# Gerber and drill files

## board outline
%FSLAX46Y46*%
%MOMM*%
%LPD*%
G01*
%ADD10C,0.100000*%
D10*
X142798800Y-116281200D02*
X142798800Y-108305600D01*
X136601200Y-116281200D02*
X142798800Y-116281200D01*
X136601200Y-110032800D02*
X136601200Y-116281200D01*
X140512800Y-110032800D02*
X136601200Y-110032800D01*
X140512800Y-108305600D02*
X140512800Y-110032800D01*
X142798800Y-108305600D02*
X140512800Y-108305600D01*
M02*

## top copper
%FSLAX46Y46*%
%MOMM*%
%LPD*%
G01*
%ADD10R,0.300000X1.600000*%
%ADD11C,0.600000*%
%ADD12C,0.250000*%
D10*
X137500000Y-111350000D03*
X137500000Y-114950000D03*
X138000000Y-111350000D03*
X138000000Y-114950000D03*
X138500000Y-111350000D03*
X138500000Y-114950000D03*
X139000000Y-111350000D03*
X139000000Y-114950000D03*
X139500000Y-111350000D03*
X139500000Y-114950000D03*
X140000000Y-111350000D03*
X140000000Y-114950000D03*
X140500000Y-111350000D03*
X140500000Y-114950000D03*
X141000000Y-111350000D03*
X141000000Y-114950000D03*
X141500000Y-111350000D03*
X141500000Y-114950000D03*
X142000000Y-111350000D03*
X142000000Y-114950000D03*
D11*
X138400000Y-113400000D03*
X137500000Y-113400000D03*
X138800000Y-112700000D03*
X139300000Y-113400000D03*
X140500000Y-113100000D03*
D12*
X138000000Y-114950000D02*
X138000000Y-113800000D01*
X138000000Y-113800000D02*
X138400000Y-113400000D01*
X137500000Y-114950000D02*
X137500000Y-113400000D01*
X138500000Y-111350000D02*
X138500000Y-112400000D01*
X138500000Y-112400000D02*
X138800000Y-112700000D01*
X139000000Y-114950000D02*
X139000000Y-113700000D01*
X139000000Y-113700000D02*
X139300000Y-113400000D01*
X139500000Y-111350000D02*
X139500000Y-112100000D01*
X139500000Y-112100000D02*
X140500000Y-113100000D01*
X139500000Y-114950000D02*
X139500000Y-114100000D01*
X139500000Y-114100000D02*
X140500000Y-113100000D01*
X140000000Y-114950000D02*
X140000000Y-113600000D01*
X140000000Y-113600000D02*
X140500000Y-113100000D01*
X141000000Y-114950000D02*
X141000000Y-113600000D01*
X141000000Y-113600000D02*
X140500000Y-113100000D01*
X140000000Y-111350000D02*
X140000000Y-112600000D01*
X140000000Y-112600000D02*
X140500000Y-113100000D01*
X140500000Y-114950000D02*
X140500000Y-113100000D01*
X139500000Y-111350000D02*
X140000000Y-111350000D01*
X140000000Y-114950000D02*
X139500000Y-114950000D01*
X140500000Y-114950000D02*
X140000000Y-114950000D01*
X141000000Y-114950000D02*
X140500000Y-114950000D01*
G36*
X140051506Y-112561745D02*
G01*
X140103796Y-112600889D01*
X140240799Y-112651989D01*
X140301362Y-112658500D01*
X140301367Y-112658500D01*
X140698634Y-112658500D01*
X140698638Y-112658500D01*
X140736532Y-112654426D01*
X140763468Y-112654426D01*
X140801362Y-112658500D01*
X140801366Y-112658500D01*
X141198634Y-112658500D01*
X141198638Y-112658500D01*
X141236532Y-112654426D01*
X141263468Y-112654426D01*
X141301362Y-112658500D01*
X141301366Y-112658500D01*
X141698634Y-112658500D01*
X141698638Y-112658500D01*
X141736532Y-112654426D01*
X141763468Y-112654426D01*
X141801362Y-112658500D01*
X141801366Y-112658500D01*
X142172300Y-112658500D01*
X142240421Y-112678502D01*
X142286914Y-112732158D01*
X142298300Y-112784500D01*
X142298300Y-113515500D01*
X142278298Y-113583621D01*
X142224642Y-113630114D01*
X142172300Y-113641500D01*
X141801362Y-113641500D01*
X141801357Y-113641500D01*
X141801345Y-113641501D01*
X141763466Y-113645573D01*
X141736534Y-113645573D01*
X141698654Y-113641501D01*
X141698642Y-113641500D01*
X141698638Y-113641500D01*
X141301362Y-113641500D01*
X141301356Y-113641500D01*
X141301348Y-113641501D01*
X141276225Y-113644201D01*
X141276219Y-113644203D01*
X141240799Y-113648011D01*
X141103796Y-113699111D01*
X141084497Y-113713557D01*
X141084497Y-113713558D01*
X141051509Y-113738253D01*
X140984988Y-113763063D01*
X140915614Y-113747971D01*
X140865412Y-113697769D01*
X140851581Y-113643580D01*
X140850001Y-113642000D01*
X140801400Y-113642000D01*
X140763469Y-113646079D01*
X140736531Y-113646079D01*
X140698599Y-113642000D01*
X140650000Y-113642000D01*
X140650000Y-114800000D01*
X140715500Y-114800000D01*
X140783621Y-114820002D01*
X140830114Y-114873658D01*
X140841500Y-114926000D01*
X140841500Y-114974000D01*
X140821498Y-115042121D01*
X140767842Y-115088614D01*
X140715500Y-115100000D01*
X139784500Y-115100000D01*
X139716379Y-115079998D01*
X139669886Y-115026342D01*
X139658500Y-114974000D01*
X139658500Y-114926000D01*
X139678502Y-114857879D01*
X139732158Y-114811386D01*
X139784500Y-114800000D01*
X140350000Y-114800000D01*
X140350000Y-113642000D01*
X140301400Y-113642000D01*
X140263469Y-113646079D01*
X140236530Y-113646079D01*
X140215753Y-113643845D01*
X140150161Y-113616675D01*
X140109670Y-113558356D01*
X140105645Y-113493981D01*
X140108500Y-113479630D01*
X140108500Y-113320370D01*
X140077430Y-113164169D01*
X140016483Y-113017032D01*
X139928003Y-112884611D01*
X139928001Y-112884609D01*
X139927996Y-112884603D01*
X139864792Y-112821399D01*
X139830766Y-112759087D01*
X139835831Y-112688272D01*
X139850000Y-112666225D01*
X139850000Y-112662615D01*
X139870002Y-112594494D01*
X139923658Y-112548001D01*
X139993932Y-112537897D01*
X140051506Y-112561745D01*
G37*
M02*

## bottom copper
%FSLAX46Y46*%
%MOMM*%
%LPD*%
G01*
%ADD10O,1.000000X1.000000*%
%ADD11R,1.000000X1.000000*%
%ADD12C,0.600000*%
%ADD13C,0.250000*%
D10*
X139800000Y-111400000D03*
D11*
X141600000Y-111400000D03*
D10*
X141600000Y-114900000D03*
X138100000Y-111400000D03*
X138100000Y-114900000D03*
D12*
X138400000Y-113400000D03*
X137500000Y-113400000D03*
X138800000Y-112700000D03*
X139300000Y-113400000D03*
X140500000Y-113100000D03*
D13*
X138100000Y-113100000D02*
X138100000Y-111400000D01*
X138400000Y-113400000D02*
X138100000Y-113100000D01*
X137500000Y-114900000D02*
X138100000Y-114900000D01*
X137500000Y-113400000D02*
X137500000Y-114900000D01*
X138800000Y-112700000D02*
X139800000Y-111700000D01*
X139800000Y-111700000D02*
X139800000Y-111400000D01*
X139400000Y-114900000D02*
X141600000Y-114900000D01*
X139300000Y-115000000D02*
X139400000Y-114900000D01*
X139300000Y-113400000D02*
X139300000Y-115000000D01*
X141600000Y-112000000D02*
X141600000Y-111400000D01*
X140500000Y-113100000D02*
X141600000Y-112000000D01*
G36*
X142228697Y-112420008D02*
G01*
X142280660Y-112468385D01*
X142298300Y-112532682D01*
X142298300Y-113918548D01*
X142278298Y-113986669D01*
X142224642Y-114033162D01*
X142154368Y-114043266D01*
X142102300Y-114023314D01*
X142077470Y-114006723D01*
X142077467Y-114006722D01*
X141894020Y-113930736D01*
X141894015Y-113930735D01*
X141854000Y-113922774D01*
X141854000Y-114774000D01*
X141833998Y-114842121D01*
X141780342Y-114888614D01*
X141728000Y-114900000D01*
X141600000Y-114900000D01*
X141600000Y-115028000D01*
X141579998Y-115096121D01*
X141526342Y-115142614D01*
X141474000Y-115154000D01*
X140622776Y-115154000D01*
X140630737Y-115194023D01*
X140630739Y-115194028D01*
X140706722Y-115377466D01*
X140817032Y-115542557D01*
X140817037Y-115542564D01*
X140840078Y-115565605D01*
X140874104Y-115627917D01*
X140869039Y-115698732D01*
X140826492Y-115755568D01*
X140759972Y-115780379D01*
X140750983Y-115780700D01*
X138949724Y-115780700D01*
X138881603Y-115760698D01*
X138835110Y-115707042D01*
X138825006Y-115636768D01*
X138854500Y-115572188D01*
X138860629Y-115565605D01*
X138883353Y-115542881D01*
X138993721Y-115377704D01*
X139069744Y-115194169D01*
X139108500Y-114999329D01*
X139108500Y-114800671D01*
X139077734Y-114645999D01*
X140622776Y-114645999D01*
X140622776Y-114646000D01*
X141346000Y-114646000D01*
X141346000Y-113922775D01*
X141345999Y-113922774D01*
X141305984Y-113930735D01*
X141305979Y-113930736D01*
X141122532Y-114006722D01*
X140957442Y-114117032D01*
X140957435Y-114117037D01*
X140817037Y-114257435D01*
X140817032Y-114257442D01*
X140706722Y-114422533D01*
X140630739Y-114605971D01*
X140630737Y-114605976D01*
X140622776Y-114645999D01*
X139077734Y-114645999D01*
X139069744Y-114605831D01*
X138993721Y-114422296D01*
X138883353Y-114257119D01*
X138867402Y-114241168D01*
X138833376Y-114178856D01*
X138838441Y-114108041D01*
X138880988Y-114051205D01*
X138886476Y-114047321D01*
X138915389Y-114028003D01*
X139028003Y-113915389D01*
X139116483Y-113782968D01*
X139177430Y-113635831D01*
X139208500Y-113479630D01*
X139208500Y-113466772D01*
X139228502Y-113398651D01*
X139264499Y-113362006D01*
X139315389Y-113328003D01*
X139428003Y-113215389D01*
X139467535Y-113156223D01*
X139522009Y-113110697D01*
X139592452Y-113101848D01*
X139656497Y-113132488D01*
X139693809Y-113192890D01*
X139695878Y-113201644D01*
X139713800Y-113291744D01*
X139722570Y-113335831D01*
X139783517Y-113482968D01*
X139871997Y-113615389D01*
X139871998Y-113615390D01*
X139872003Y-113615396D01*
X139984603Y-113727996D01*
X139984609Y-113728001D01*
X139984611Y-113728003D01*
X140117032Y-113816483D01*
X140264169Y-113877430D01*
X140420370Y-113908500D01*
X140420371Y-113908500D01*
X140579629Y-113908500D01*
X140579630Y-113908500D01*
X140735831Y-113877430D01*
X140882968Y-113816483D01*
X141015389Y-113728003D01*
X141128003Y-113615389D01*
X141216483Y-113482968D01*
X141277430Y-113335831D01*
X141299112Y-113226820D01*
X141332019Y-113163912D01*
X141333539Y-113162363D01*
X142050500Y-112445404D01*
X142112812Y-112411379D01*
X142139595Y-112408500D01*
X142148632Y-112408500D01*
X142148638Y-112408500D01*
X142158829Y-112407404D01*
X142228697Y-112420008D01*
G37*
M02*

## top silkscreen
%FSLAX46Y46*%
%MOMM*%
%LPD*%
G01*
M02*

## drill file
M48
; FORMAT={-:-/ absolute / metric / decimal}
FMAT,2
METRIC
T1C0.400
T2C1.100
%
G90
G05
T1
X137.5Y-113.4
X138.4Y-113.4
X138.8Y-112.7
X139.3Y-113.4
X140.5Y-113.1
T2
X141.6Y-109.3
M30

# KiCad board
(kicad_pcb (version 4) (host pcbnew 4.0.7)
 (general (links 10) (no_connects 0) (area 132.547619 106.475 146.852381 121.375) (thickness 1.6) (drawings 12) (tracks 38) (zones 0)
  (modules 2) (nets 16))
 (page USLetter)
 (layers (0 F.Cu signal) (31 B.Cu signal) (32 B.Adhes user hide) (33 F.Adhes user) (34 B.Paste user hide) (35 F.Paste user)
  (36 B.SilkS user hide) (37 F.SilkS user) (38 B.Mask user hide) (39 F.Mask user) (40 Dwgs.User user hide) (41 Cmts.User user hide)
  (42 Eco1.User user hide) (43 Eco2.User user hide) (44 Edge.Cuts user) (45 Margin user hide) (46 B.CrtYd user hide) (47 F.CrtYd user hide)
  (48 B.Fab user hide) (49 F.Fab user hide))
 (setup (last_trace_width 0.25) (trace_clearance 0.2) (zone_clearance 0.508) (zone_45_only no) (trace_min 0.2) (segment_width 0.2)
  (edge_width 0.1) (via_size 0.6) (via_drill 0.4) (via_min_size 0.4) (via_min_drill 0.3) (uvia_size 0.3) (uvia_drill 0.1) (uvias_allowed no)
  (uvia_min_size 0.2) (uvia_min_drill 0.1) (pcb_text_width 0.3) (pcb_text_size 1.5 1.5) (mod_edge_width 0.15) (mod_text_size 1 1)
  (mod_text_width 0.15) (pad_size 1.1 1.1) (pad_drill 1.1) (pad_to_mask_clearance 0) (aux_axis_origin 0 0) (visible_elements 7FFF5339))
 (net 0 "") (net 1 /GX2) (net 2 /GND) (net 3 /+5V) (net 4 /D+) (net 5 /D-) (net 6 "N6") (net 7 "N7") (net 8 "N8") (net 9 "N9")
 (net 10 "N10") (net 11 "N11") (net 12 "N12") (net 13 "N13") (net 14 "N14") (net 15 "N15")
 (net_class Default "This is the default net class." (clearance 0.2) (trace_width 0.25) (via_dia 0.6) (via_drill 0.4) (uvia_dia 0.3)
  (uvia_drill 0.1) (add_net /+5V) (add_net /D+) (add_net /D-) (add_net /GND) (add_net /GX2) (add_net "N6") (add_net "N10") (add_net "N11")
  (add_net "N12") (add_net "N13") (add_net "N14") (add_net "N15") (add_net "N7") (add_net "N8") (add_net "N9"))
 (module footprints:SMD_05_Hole (layer B.Cu) (at 139.6 113.9)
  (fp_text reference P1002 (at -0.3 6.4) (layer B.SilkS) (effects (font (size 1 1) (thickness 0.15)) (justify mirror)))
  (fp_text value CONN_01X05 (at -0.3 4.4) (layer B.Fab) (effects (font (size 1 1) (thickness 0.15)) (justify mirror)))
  (pad 5 smd oval (at 0.2 -2.5) (size 1 1) (layers B.Cu B.Paste B.Mask) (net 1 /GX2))
  (pad 1 smd rect (at 2 -2.5) (size 1 1) (layers B.Cu B.Paste B.Mask) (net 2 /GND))
  (pad 2 smd oval (at 2 1) (size 1 1) (layers B.Cu B.Paste B.Mask) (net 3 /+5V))
  (pad 3 smd oval (at -1.5 -2.5) (size 1 1) (layers B.Cu B.Paste B.Mask) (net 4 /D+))
  (pad 4 smd oval (at -1.5 1) (size 1 1) (layers B.Cu B.Paste B.Mask) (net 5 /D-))
  (pad "" np_thru_hole circle (at 2 -4.6) (size 1.1 1.1) (drill 1.1) (layers *.Cu *.Mask B.SilkS)))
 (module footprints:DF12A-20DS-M (layer F.Cu) (at 139.7 107.95)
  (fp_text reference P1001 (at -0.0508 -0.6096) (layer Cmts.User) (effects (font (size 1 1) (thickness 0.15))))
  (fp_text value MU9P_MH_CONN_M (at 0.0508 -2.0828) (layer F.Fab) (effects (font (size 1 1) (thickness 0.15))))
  (pad 1 smd rect (at -2.2 3.4) (size 0.3 1.6) (layers F.Cu F.Paste F.Mask) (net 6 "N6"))
  (pad 2 smd rect (at -2.2 7) (size 0.3 1.6) (layers F.Cu F.Paste F.Mask) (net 5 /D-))
  (pad 3 smd rect (at -1.7 3.4) (size 0.3 1.6) (layers F.Cu F.Paste F.Mask) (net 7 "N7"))
  (pad 4 smd rect (at -1.7 7) (size 0.3 1.6) (layers F.Cu F.Paste F.Mask) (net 4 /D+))
  (pad 5 smd rect (at -1.2 3.4) (size 0.3 1.6) (layers F.Cu F.Paste F.Mask) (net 1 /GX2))
  (pad 6 smd rect (at -1.2 7) (size 0.3 1.6) (layers F.Cu F.Paste F.Mask) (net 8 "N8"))
  (pad 7 smd rect (at -0.7 3.4) (size 0.3 1.6) (layers F.Cu F.Paste F.Mask) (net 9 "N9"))
  (pad 8 smd rect (at -0.7 7) (size 0.3 1.6) (layers F.Cu F.Paste F.Mask) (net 3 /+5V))
  (pad 9 smd rect (at -0.2 3.4) (size 0.3 1.6) (layers F.Cu F.Paste F.Mask) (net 2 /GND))
  (pad 10 smd rect (at -0.2 7) (size 0.3 1.6) (layers F.Cu F.Paste F.Mask) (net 2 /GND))
  (pad 11 smd rect (at 0.3 3.4) (size 0.3 1.6) (layers F.Cu F.Paste F.Mask) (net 2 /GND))
  (pad 12 smd rect (at 0.3 7) (size 0.3 1.6) (layers F.Cu F.Paste F.Mask) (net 2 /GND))
  (pad 13 smd rect (at 0.8 3.4) (size 0.3 1.6) (layers F.Cu F.Paste F.Mask) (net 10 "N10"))
  (pad 14 smd rect (at 0.8 7) (size 0.3 1.6) (layers F.Cu F.Paste F.Mask) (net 2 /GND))
  (pad 15 smd rect (at 1.3 3.4) (size 0.3 1.6) (layers F.Cu F.Paste F.Mask) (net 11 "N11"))
  (pad 16 smd rect (at 1.3 7) (size 0.3 1.6) (layers F.Cu F.Paste F.Mask) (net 2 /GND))
  (pad 17 smd rect (at 1.8 3.4) (size 0.3 1.6) (layers F.Cu F.Paste F.Mask) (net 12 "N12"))
  (pad 18 smd rect (at 1.8 7) (size 0.3 1.6) (layers F.Cu F.Paste F.Mask) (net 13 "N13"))
  (pad 19 smd rect (at 2.3 3.4) (size 0.3 1.6) (layers F.Cu F.Paste F.Mask) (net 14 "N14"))
  (pad 20 smd rect (at 2.3 7) (size 0.3 1.6) (layers F.Cu F.Paste F.Mask) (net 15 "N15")))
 (gr_line (start 142.7988 116.2812) (end 142.7988 108.3056) (angle 90) (layer Edge.Cuts) (width 0.1))
 (gr_line (start 136.6012 116.2812) (end 142.7988 116.2812) (angle 90) (layer Edge.Cuts) (width 0.1))
 (gr_line (start 136.6012 110.0328) (end 136.6012 116.2812) (angle 90) (layer Edge.Cuts) (width 0.1))
 (gr_line (start 140.5128 110.0328) (end 136.6012 110.0328) (angle 90) (layer Edge.Cuts) (width 0.1))
 (gr_line (start 140.5128 108.3056) (end 140.5128 110.0328) (angle 90) (layer Edge.Cuts) (width 0.1))
 (gr_line (start 142.7988 108.3056) (end 140.5128 108.3056) (angle 90) (layer Edge.Cuts) (width 0.1))
 (segment (start 138 114.95) (end 138 113.8) (width 0.25) (layer F.Cu) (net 4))
 (segment (start 138.1 113.1) (end 138.1 111.4) (width 0.25) (layer B.Cu) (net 4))
 (segment (start 138.4 113.4) (end 138.1 113.1) (width 0.25) (layer B.Cu) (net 4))
 (via (at 138.4 113.4) (size 0.6) (drill 0.4) (layers F.Cu B.Cu) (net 4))
 (segment (start 138 113.8) (end 138.4 113.4) (width 0.25) (layer F.Cu) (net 4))
 (segment (start 137.5 114.95) (end 137.5 113.4) (width 0.25) (layer F.Cu) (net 5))
 (segment (start 137.5 114.9) (end 138.1 114.9) (width 0.25) (layer B.Cu) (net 5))
 (segment (start 137.5 113.4) (end 137.5 114.9) (width 0.25) (layer B.Cu) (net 5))
 (via (at 137.5 113.4) (size 0.6) (drill 0.4) (layers F.Cu B.Cu) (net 5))
 (segment (start 138.5 111.35) (end 138.5 112.4) (width 0.25) (layer F.Cu) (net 1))
 (segment (start 138.8 112.7) (end 139.8 111.7) (width 0.25) (layer B.Cu) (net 1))
 (via (at 138.8 112.7) (size 0.6) (drill 0.4) (layers F.Cu B.Cu) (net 1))
 (segment (start 138.5 112.4) (end 138.8 112.7) (width 0.25) (layer F.Cu) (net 1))
 (segment (start 139.8 111.7) (end 139.8 111.4) (width 0.25) (layer B.Cu) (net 1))
 (segment (start 139 114.95) (end 139 113.7) (width 0.25) (layer F.Cu) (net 3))
 (segment (start 139.4 114.9) (end 141.6 114.9) (width 0.25) (layer B.Cu) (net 3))
 (segment (start 139.3 115) (end 139.4 114.9) (width 0.25) (layer B.Cu) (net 3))
 (segment (start 139.3 113.4) (end 139.3 115) (width 0.25) (layer B.Cu) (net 3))
 (via (at 139.3 113.4) (size 0.6) (drill 0.4) (layers F.Cu B.Cu) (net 3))
 (segment (start 139 113.7) (end 139.3 113.4) (width 0.25) (layer F.Cu) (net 3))
 (segment (start 139.5 111.35) (end 139.5 112.1) (width 0.25) (layer F.Cu) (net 2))
 (segment (start 139.5 112.1) (end 140.5 113.1) (width 0.25) (layer F.Cu) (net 2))
 (segment (start 139.5 114.95) (end 139.5 114.1) (width 0.25) (layer F.Cu) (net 2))
 (segment (start 139.5 114.1) (end 140.5 113.1) (width 0.25) (layer F.Cu) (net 2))
 (segment (start 140 114.95) (end 140 113.6) (width 0.25) (layer F.Cu) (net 2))
 (segment (start 140 113.6) (end 140.5 113.1) (width 0.25) (layer F.Cu) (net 2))
 (segment (start 141 114.95) (end 141 113.6) (width 0.25) (layer F.Cu) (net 2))
 (segment (start 141 113.6) (end 140.5 113.1) (width 0.25) (layer F.Cu) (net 2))
 (segment (start 140 111.35) (end 140 112.6) (width 0.25) (layer F.Cu) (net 2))
 (segment (start 140 112.6) (end 140.5 113.1) (width 0.25) (layer F.Cu) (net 2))
 (segment (start 140.5 114.95) (end 140.5 113.1) (width 0.25) (layer F.Cu) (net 2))
 (segment (start 141.6 112) (end 141.6 111.4) (width 0.25) (layer B.Cu) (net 2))
 (segment (start 140.5 113.1) (end 141.6 112) (width 0.25) (layer B.Cu) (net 2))
 (via (at 140.5 113.1) (size 0.6) (drill 0.4) (layers F.Cu B.Cu) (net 2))
 (segment (start 139.5 111.35) (end 140 111.35) (width 0.25) (layer F.Cu) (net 2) (status 30))
 (segment (start 140 114.95) (end 139.5 114.95) (width 0.25) (layer F.Cu) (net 2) (status 30))
 (segment (start 140.5 114.95) (end 140 114.95) (width 0.25) (layer F.Cu) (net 2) (status 30))
 (segment (start 141 114.95) (end 140.5 114.95) (width 0.25) (layer F.Cu) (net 2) (status 30))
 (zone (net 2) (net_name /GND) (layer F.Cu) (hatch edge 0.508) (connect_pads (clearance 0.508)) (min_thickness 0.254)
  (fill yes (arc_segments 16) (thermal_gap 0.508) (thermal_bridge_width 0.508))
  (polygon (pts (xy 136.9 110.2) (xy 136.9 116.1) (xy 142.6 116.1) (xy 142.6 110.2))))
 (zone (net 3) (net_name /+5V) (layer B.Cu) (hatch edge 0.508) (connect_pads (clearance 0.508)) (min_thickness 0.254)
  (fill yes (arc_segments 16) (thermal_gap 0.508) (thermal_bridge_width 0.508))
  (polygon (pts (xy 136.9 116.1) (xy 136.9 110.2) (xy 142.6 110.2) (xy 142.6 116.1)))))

